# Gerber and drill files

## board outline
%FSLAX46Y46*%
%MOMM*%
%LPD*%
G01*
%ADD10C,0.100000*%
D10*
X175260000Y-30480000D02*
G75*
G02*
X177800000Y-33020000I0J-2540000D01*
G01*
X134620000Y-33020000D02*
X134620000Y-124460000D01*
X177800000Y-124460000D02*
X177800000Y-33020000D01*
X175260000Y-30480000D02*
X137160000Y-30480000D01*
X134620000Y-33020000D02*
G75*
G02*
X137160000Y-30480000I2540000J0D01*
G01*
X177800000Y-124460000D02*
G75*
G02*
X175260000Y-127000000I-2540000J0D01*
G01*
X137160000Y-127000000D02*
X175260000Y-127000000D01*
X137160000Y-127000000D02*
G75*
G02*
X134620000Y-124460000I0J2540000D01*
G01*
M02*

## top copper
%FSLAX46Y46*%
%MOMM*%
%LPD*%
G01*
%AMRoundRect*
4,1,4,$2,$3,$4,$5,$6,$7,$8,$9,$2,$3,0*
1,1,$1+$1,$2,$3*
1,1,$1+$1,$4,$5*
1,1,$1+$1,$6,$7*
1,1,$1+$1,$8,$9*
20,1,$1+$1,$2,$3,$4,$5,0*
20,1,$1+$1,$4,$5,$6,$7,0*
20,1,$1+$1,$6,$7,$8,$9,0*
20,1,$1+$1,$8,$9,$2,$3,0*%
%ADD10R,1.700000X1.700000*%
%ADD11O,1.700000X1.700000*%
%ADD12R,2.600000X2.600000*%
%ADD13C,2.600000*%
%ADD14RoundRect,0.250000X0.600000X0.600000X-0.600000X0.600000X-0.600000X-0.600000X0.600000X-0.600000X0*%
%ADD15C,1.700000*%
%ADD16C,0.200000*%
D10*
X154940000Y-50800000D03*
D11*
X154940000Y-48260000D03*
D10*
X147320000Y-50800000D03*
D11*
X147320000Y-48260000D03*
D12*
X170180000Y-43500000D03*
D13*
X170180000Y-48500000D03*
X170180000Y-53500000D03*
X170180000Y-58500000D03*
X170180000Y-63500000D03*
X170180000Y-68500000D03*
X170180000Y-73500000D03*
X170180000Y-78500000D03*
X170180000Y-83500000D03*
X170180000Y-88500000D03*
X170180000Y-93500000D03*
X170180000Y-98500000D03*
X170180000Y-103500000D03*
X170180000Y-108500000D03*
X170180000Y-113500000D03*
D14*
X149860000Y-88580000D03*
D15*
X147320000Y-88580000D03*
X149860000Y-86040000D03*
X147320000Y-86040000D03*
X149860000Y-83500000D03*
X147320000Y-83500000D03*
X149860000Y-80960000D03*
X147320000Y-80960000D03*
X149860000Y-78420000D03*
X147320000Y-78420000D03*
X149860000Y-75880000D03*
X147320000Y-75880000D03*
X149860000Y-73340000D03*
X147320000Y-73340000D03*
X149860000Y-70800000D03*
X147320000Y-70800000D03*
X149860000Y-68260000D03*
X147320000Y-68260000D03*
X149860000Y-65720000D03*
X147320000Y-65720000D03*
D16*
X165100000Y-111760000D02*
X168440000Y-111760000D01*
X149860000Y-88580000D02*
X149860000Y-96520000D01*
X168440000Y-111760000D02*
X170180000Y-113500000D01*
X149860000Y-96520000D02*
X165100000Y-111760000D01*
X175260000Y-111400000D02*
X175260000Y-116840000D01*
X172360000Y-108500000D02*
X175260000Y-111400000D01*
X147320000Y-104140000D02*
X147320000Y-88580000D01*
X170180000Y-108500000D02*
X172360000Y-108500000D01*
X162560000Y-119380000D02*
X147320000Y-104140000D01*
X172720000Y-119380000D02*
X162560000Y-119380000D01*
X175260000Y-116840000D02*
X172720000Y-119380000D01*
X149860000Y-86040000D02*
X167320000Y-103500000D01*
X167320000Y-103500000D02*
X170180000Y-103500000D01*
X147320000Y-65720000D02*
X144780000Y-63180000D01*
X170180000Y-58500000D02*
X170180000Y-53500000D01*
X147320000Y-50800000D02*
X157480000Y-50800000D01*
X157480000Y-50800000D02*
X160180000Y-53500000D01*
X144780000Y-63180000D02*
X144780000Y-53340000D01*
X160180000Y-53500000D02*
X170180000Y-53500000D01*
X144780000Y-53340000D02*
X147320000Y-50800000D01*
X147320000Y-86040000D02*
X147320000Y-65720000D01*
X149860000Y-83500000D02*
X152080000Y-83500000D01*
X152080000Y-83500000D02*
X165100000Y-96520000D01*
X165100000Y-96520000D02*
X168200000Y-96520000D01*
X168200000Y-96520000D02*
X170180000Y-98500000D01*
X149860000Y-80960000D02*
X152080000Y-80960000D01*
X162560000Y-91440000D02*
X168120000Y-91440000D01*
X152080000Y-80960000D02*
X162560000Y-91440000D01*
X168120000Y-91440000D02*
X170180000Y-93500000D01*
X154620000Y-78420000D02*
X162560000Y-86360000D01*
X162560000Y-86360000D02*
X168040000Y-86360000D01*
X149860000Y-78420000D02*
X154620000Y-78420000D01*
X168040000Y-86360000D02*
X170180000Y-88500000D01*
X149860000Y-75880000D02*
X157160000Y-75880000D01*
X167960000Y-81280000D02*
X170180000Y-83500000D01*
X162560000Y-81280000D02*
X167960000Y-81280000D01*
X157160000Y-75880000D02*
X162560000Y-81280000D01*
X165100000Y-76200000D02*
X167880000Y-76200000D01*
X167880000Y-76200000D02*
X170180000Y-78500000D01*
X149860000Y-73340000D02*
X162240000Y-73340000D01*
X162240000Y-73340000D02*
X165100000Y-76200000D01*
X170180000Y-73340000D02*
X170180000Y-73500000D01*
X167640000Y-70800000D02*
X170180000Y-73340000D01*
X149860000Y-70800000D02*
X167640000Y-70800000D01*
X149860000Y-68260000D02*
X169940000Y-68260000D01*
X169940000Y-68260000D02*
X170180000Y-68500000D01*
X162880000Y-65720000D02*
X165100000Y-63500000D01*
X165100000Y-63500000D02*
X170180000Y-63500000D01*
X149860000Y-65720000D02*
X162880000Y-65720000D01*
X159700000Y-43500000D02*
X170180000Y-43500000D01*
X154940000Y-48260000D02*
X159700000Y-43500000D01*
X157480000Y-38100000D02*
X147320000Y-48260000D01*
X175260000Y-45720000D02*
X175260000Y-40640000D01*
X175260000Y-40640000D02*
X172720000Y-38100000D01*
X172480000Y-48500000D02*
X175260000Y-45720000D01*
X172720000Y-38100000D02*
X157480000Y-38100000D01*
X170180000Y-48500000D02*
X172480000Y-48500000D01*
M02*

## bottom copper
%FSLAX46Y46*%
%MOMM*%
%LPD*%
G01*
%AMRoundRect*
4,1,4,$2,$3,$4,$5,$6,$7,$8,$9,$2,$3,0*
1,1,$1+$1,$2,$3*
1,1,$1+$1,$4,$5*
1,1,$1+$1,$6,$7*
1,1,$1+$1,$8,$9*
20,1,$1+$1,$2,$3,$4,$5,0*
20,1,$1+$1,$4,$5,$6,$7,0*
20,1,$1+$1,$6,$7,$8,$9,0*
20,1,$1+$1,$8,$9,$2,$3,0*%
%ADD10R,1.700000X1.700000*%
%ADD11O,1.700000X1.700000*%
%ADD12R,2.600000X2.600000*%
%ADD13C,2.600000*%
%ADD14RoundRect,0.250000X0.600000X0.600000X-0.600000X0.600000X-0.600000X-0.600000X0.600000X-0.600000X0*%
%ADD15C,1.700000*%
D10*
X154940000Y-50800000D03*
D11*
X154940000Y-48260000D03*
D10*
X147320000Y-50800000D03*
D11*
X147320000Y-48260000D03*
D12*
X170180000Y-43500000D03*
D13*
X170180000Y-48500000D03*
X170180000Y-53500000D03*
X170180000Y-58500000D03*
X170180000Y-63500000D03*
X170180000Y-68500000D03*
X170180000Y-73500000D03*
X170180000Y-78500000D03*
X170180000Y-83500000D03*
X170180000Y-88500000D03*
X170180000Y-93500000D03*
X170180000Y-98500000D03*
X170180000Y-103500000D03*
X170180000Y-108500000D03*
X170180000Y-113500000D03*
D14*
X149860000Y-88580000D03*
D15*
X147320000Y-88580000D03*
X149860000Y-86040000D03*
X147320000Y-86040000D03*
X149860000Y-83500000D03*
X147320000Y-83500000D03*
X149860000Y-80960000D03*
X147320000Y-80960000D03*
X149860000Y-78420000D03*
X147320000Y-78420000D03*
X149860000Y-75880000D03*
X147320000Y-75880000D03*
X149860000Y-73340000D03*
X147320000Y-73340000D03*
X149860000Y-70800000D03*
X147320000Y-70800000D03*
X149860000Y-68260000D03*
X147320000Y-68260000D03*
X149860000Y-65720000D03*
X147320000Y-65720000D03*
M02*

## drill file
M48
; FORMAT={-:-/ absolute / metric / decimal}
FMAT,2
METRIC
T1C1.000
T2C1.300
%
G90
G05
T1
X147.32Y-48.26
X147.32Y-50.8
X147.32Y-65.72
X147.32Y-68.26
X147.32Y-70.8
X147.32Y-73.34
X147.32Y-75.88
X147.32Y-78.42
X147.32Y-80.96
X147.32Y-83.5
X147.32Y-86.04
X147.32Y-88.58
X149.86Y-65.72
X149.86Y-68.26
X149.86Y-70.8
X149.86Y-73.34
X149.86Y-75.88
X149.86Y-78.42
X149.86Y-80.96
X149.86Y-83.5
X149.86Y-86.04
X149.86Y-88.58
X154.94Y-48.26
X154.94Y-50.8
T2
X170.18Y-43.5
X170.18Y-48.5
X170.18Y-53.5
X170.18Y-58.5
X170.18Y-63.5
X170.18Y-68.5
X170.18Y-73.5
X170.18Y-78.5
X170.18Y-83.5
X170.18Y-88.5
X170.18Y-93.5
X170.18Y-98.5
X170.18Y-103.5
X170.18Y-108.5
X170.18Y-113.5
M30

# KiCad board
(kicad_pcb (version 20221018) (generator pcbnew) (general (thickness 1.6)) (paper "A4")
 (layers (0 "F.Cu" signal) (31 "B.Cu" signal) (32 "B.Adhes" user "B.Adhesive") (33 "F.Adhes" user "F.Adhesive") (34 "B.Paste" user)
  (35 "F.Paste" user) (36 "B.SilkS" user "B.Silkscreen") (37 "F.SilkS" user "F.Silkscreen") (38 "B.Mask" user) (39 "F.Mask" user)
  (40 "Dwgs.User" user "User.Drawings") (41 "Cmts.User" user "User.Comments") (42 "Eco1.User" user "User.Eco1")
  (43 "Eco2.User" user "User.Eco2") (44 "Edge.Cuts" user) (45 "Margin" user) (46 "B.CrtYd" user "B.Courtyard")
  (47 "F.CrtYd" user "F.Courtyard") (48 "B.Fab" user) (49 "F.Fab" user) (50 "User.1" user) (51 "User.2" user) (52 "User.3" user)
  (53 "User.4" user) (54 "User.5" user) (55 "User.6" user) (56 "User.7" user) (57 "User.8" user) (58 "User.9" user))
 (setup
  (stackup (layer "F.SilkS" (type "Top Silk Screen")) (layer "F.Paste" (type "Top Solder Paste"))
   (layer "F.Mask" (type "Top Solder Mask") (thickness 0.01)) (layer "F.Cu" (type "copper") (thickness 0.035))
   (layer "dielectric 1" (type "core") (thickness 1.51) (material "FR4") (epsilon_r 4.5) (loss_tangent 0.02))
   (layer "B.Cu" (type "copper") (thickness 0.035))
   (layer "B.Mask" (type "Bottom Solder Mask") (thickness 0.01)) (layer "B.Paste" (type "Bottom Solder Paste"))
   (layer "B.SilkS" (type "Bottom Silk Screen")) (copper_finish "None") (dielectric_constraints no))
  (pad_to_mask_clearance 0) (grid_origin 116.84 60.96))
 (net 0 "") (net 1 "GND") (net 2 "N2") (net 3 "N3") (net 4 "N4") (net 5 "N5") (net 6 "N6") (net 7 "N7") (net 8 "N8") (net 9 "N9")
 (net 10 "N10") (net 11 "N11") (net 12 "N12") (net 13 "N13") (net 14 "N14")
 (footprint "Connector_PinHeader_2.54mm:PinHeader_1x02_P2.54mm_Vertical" (layer "F.Cu") (at 154.94 50.8 180)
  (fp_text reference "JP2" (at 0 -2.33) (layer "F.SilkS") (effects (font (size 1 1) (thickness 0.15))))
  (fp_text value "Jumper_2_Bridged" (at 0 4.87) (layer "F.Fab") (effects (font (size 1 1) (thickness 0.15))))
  (pad "1" thru_hole rect (at 0 0 180) (size 1.7 1.7) (drill 1) (layers "*.Cu" "*.Mask") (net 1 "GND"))
  (pad "2" thru_hole oval (at 0 2.54 180) (size 1.7 1.7) (drill 1) (layers "*.Cu" "*.Mask") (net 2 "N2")))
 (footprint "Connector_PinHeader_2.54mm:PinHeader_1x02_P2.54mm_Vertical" (layer "F.Cu") (at 147.32 50.8 180)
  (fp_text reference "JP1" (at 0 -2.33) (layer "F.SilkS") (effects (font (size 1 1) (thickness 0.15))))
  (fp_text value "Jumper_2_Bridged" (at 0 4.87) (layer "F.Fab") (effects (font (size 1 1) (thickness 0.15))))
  (pad "1" thru_hole rect (at 0 0 180) (size 1.7 1.7) (drill 1) (layers "*.Cu" "*.Mask") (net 1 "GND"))
  (pad "2" thru_hole oval (at 0 2.54 180) (size 1.7 1.7) (drill 1) (layers "*.Cu" "*.Mask") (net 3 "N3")))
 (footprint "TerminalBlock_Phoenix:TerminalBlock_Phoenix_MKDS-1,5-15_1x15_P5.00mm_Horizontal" (layer "F.Cu") (at 170.18 43.5 -90)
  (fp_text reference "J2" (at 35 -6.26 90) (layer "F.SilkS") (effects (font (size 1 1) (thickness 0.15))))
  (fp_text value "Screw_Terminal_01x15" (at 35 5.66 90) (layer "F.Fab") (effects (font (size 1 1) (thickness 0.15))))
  (pad "1" thru_hole rect (at 0 0 270) (size 2.6 2.6) (drill 1.3) (layers "*.Cu" "*.Mask") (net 2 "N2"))
  (pad "2" thru_hole circle (at 5 0 270) (size 2.6 2.6) (drill 1.3) (layers "*.Cu" "*.Mask") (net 3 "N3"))
  (pad "3" thru_hole circle (at 10 0 270) (size 2.6 2.6) (drill 1.3) (layers "*.Cu" "*.Mask") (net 1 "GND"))
  (pad "4" thru_hole circle (at 15 0 270) (size 2.6 2.6) (drill 1.3) (layers "*.Cu" "*.Mask") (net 1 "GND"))
  (pad "5" thru_hole circle (at 20 0 270) (size 2.6 2.6) (drill 1.3) (layers "*.Cu" "*.Mask") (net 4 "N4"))
  (pad "6" thru_hole circle (at 25 0 270) (size 2.6 2.6) (drill 1.3) (layers "*.Cu" "*.Mask") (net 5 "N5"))
  (pad "7" thru_hole circle (at 30 0 270) (size 2.6 2.6) (drill 1.3) (layers "*.Cu" "*.Mask") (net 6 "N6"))
  (pad "8" thru_hole circle (at 35 0 270) (size 2.6 2.6) (drill 1.3) (layers "*.Cu" "*.Mask") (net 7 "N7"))
  (pad "9" thru_hole circle (at 40 0 270) (size 2.6 2.6) (drill 1.3) (layers "*.Cu" "*.Mask") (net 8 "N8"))
  (pad "10" thru_hole circle (at 45 0 270) (size 2.6 2.6) (drill 1.3) (layers "*.Cu" "*.Mask") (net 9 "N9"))
  (pad "11" thru_hole circle (at 50 0 270) (size 2.6 2.6) (drill 1.3) (layers "*.Cu" "*.Mask") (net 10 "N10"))
  (pad "12" thru_hole circle (at 55 0 270) (size 2.6 2.6) (drill 1.3) (layers "*.Cu" "*.Mask") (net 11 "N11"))
  (pad "13" thru_hole circle (at 60 0 270) (size 2.6 2.6) (drill 1.3) (layers "*.Cu" "*.Mask") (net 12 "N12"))
  (pad "14" thru_hole circle (at 65 0 270) (size 2.6 2.6) (drill 1.3) (layers "*.Cu" "*.Mask") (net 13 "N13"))
  (pad "15" thru_hole circle (at 70 0 270) (size 2.6 2.6) (drill 1.3) (layers "*.Cu" "*.Mask") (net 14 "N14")))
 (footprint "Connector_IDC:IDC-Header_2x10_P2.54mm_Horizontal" (layer "F.Cu") (at 149.86 88.58 180)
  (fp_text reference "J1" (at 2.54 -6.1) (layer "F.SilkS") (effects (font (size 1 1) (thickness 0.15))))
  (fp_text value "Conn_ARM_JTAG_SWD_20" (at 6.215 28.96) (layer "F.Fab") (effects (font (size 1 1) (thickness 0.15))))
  (pad "1" thru_hole roundrect (at 0 0 180) (size 1.7 1.7) (drill 1) (layers "*.Cu" "*.Mask") (roundrect_rratio 0.1470588235) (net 14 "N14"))
  (pad "2" thru_hole circle (at 2.54 0 180) (size 1.7 1.7) (drill 1) (layers "*.Cu" "*.Mask") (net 13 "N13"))
  (pad "3" thru_hole circle (at 0 2.54 180) (size 1.7 1.7) (drill 1) (layers "*.Cu" "*.Mask") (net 12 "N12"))
  (pad "4" thru_hole circle (at 2.54 2.54 180) (size 1.7 1.7) (drill 1) (layers "*.Cu" "*.Mask") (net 1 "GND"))
  (pad "5" thru_hole circle (at 0 5.08 180) (size 1.7 1.7) (drill 1) (layers "*.Cu" "*.Mask") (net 11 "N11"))
  (pad "6" thru_hole circle (at 2.54 5.08 180) (size 1.7 1.7) (drill 1) (layers "*.Cu" "*.Mask") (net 1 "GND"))
  (pad "7" thru_hole circle (at 0 7.62 180) (size 1.7 1.7) (drill 1) (layers "*.Cu" "*.Mask") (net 10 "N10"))
  (pad "8" thru_hole circle (at 2.54 7.62 180) (size 1.7 1.7) (drill 1) (layers "*.Cu" "*.Mask") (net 1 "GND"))
  (pad "9" thru_hole circle (at 0 10.16 180) (size 1.7 1.7) (drill 1) (layers "*.Cu" "*.Mask") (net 9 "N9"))
  (pad "10" thru_hole circle (at 2.54 10.16 180) (size 1.7 1.7) (drill 1) (layers "*.Cu" "*.Mask") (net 1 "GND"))
  (pad "11" thru_hole circle (at 0 12.7 180) (size 1.7 1.7) (drill 1) (layers "*.Cu" "*.Mask") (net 8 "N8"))
  (pad "12" thru_hole circle (at 2.54 12.7 180) (size 1.7 1.7) (drill 1) (layers "*.Cu" "*.Mask") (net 1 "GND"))
  (pad "13" thru_hole circle (at 0 15.24 180) (size 1.7 1.7) (drill 1) (layers "*.Cu" "*.Mask") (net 7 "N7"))
  (pad "14" thru_hole circle (at 2.54 15.24 180) (size 1.7 1.7) (drill 1) (layers "*.Cu" "*.Mask") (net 1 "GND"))
  (pad "15" thru_hole circle (at 0 17.78 180) (size 1.7 1.7) (drill 1) (layers "*.Cu" "*.Mask") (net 6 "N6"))
  (pad "16" thru_hole circle (at 2.54 17.78 180) (size 1.7 1.7) (drill 1) (layers "*.Cu" "*.Mask") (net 1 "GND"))
  (pad "17" thru_hole circle (at 0 20.32 180) (size 1.7 1.7) (drill 1) (layers "*.Cu" "*.Mask") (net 5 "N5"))
  (pad "18" thru_hole circle (at 2.54 20.32 180) (size 1.7 1.7) (drill 1) (layers "*.Cu" "*.Mask") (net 1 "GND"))
  (pad "19" thru_hole circle (at 0 22.86 180) (size 1.7 1.7) (drill 1) (layers "*.Cu" "*.Mask") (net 4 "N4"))
  (pad "20" thru_hole circle (at 2.54 22.86 180) (size 1.7 1.7) (drill 1) (layers "*.Cu" "*.Mask") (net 1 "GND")))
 (gr_arc (start 175.26 30.48) (mid 177.056051 31.223949) (end 177.8 33.02) (stroke (width 0.1) (type default)) (layer "Edge.Cuts"))
 (gr_line (start 134.62 33.02) (end 134.62 124.46) (stroke (width 0.1) (type default)) (layer "Edge.Cuts"))
 (gr_line (start 177.8 124.46) (end 177.8 33.02) (stroke (width 0.1) (type default)) (layer "Edge.Cuts"))
 (gr_line (start 175.26 30.48) (end 137.16 30.48) (stroke (width 0.1) (type default)) (layer "Edge.Cuts"))
 (gr_arc (start 134.62 33.02) (mid 135.363949 31.223949) (end 137.16 30.48) (stroke (width 0.1) (type default)) (layer "Edge.Cuts"))
 (gr_arc (start 177.8 124.46) (mid 177.056051 126.256051) (end 175.26 127) (stroke (width 0.1) (type default)) (layer "Edge.Cuts"))
 (gr_line (start 137.16 127) (end 175.26 127) (stroke (width 0.1) (type default)) (layer "Edge.Cuts"))
 (gr_arc (start 137.16 127) (mid 135.363949 126.256051) (end 134.62 124.46) (stroke (width 0.1) (type default)) (layer "Edge.Cuts"))
 (segment (start 165.1 111.76) (end 168.44 111.76) (width 0.2) (layer "F.Cu") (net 14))
 (segment (start 149.86 88.58) (end 149.86 96.52) (width 0.2) (layer "F.Cu") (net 14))
 (segment (start 168.44 111.76) (end 170.18 113.5) (width 0.2) (layer "F.Cu") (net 14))
 (segment (start 149.86 96.52) (end 165.1 111.76) (width 0.2) (layer "F.Cu") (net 14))
 (segment (start 175.26 111.4) (end 175.26 116.84) (width 0.2) (layer "F.Cu") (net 13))
 (segment (start 172.36 108.5) (end 175.26 111.4) (width 0.2) (layer "F.Cu") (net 13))
 (segment (start 147.32 104.14) (end 147.32 88.58) (width 0.2) (layer "F.Cu") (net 13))
 (segment (start 170.18 108.5) (end 172.36 108.5) (width 0.2) (layer "F.Cu") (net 13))
 (segment (start 162.56 119.38) (end 147.32 104.14) (width 0.2) (layer "F.Cu") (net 13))
 (segment (start 172.72 119.38) (end 162.56 119.38) (width 0.2) (layer "F.Cu") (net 13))
 (segment (start 175.26 116.84) (end 172.72 119.38) (width 0.2) (layer "F.Cu") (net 13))
 (segment (start 149.86 86.04) (end 167.32 103.5) (width 0.2) (layer "F.Cu") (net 12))
 (segment (start 167.32 103.5) (end 170.18 103.5) (width 0.2) (layer "F.Cu") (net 12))
 (segment (start 147.32 65.72) (end 144.78 63.18) (width 0.2) (layer "F.Cu") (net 1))
 (segment (start 170.18 58.5) (end 170.18 53.5) (width 0.2) (layer "F.Cu") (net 1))
 (segment (start 147.32 50.8) (end 157.48 50.8) (width 0.2) (layer "F.Cu") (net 1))
 (segment (start 157.48 50.8) (end 160.18 53.5) (width 0.2) (layer "F.Cu") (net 1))
 (segment (start 144.78 63.18) (end 144.78 53.34) (width 0.2) (layer "F.Cu") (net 1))
 (segment (start 160.18 53.5) (end 170.18 53.5) (width 0.2) (layer "F.Cu") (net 1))
 (segment (start 144.78 53.34) (end 147.32 50.8) (width 0.2) (layer "F.Cu") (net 1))
 (segment (start 147.32 86.04) (end 147.32 65.72) (width 0.2) (layer "F.Cu") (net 1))
 (segment (start 149.86 83.5) (end 152.08 83.5) (width 0.2) (layer "F.Cu") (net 11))
 (segment (start 152.08 83.5) (end 165.1 96.52) (width 0.2) (layer "F.Cu") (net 11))
 (segment (start 165.1 96.52) (end 168.2 96.52) (width 0.2) (layer "F.Cu") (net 11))
 (segment (start 168.2 96.52) (end 170.18 98.5) (width 0.2) (layer "F.Cu") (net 11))
 (segment (start 149.86 80.96) (end 152.08 80.96) (width 0.2) (layer "F.Cu") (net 10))
 (segment (start 162.56 91.44) (end 168.12 91.44) (width 0.2) (layer "F.Cu") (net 10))
 (segment (start 152.08 80.96) (end 162.56 91.44) (width 0.2) (layer "F.Cu") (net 10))
 (segment (start 168.12 91.44) (end 170.18 93.5) (width 0.2) (layer "F.Cu") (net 10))
 (segment (start 154.62 78.42) (end 162.56 86.36) (width 0.2) (layer "F.Cu") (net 9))
 (segment (start 162.56 86.36) (end 168.04 86.36) (width 0.2) (layer "F.Cu") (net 9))
 (segment (start 149.86 78.42) (end 154.62 78.42) (width 0.2) (layer "F.Cu") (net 9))
 (segment (start 168.04 86.36) (end 170.18 88.5) (width 0.2) (layer "F.Cu") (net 9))
 (segment (start 149.86 75.88) (end 157.16 75.88) (width 0.2) (layer "F.Cu") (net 8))
 (segment (start 167.96 81.28) (end 170.18 83.5) (width 0.2) (layer "F.Cu") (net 8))
 (segment (start 162.56 81.28) (end 167.96 81.28) (width 0.2) (layer "F.Cu") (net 8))
 (segment (start 157.16 75.88) (end 162.56 81.28) (width 0.2) (layer "F.Cu") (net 8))
 (segment (start 165.1 76.2) (end 167.88 76.2) (width 0.2) (layer "F.Cu") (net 7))
 (segment (start 167.88 76.2) (end 170.18 78.5) (width 0.2) (layer "F.Cu") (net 7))
 (segment (start 149.86 73.34) (end 162.24 73.34) (width 0.2) (layer "F.Cu") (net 7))
 (segment (start 162.24 73.34) (end 165.1 76.2) (width 0.2) (layer "F.Cu") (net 7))
 (segment (start 170.18 73.34) (end 170.18 73.5) (width 0.2) (layer "F.Cu") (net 6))
 (segment (start 167.64 70.8) (end 170.18 73.34) (width 0.2) (layer "F.Cu") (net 6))
 (segment (start 149.86 70.8) (end 167.64 70.8) (width 0.2) (layer "F.Cu") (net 6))
 (segment (start 149.86 68.26) (end 169.94 68.26) (width 0.2) (layer "F.Cu") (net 5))
 (segment (start 169.94 68.26) (end 170.18 68.5) (width 0.2) (layer "F.Cu") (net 5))
 (segment (start 162.88 65.72) (end 165.1 63.5) (width 0.2) (layer "F.Cu") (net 4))
 (segment (start 165.1 63.5) (end 170.18 63.5) (width 0.2) (layer "F.Cu") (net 4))
 (segment (start 149.86 65.72) (end 162.88 65.72) (width 0.2) (layer "F.Cu") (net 4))
 (segment (start 159.7 43.5) (end 170.18 43.5) (width 0.2) (layer "F.Cu") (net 2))
 (segment (start 154.94 48.26) (end 159.7 43.5) (width 0.2) (layer "F.Cu") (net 2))
 (segment (start 157.48 38.1) (end 147.32 48.26) (width 0.2) (layer "F.Cu") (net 3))
 (segment (start 175.26 45.72) (end 175.26 40.64) (width 0.2) (layer "F.Cu") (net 3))
 (segment (start 175.26 40.64) (end 172.72 38.1) (width 0.2) (layer "F.Cu") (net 3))
 (segment (start 172.48 48.5) (end 175.26 45.72) (width 0.2) (layer "F.Cu") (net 3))
 (segment (start 172.72 38.1) (end 157.48 38.1) (width 0.2) (layer "F.Cu") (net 3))
 (segment (start 170.18 48.5) (end 172.48 48.5) (width 0.2) (layer "F.Cu") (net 3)))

